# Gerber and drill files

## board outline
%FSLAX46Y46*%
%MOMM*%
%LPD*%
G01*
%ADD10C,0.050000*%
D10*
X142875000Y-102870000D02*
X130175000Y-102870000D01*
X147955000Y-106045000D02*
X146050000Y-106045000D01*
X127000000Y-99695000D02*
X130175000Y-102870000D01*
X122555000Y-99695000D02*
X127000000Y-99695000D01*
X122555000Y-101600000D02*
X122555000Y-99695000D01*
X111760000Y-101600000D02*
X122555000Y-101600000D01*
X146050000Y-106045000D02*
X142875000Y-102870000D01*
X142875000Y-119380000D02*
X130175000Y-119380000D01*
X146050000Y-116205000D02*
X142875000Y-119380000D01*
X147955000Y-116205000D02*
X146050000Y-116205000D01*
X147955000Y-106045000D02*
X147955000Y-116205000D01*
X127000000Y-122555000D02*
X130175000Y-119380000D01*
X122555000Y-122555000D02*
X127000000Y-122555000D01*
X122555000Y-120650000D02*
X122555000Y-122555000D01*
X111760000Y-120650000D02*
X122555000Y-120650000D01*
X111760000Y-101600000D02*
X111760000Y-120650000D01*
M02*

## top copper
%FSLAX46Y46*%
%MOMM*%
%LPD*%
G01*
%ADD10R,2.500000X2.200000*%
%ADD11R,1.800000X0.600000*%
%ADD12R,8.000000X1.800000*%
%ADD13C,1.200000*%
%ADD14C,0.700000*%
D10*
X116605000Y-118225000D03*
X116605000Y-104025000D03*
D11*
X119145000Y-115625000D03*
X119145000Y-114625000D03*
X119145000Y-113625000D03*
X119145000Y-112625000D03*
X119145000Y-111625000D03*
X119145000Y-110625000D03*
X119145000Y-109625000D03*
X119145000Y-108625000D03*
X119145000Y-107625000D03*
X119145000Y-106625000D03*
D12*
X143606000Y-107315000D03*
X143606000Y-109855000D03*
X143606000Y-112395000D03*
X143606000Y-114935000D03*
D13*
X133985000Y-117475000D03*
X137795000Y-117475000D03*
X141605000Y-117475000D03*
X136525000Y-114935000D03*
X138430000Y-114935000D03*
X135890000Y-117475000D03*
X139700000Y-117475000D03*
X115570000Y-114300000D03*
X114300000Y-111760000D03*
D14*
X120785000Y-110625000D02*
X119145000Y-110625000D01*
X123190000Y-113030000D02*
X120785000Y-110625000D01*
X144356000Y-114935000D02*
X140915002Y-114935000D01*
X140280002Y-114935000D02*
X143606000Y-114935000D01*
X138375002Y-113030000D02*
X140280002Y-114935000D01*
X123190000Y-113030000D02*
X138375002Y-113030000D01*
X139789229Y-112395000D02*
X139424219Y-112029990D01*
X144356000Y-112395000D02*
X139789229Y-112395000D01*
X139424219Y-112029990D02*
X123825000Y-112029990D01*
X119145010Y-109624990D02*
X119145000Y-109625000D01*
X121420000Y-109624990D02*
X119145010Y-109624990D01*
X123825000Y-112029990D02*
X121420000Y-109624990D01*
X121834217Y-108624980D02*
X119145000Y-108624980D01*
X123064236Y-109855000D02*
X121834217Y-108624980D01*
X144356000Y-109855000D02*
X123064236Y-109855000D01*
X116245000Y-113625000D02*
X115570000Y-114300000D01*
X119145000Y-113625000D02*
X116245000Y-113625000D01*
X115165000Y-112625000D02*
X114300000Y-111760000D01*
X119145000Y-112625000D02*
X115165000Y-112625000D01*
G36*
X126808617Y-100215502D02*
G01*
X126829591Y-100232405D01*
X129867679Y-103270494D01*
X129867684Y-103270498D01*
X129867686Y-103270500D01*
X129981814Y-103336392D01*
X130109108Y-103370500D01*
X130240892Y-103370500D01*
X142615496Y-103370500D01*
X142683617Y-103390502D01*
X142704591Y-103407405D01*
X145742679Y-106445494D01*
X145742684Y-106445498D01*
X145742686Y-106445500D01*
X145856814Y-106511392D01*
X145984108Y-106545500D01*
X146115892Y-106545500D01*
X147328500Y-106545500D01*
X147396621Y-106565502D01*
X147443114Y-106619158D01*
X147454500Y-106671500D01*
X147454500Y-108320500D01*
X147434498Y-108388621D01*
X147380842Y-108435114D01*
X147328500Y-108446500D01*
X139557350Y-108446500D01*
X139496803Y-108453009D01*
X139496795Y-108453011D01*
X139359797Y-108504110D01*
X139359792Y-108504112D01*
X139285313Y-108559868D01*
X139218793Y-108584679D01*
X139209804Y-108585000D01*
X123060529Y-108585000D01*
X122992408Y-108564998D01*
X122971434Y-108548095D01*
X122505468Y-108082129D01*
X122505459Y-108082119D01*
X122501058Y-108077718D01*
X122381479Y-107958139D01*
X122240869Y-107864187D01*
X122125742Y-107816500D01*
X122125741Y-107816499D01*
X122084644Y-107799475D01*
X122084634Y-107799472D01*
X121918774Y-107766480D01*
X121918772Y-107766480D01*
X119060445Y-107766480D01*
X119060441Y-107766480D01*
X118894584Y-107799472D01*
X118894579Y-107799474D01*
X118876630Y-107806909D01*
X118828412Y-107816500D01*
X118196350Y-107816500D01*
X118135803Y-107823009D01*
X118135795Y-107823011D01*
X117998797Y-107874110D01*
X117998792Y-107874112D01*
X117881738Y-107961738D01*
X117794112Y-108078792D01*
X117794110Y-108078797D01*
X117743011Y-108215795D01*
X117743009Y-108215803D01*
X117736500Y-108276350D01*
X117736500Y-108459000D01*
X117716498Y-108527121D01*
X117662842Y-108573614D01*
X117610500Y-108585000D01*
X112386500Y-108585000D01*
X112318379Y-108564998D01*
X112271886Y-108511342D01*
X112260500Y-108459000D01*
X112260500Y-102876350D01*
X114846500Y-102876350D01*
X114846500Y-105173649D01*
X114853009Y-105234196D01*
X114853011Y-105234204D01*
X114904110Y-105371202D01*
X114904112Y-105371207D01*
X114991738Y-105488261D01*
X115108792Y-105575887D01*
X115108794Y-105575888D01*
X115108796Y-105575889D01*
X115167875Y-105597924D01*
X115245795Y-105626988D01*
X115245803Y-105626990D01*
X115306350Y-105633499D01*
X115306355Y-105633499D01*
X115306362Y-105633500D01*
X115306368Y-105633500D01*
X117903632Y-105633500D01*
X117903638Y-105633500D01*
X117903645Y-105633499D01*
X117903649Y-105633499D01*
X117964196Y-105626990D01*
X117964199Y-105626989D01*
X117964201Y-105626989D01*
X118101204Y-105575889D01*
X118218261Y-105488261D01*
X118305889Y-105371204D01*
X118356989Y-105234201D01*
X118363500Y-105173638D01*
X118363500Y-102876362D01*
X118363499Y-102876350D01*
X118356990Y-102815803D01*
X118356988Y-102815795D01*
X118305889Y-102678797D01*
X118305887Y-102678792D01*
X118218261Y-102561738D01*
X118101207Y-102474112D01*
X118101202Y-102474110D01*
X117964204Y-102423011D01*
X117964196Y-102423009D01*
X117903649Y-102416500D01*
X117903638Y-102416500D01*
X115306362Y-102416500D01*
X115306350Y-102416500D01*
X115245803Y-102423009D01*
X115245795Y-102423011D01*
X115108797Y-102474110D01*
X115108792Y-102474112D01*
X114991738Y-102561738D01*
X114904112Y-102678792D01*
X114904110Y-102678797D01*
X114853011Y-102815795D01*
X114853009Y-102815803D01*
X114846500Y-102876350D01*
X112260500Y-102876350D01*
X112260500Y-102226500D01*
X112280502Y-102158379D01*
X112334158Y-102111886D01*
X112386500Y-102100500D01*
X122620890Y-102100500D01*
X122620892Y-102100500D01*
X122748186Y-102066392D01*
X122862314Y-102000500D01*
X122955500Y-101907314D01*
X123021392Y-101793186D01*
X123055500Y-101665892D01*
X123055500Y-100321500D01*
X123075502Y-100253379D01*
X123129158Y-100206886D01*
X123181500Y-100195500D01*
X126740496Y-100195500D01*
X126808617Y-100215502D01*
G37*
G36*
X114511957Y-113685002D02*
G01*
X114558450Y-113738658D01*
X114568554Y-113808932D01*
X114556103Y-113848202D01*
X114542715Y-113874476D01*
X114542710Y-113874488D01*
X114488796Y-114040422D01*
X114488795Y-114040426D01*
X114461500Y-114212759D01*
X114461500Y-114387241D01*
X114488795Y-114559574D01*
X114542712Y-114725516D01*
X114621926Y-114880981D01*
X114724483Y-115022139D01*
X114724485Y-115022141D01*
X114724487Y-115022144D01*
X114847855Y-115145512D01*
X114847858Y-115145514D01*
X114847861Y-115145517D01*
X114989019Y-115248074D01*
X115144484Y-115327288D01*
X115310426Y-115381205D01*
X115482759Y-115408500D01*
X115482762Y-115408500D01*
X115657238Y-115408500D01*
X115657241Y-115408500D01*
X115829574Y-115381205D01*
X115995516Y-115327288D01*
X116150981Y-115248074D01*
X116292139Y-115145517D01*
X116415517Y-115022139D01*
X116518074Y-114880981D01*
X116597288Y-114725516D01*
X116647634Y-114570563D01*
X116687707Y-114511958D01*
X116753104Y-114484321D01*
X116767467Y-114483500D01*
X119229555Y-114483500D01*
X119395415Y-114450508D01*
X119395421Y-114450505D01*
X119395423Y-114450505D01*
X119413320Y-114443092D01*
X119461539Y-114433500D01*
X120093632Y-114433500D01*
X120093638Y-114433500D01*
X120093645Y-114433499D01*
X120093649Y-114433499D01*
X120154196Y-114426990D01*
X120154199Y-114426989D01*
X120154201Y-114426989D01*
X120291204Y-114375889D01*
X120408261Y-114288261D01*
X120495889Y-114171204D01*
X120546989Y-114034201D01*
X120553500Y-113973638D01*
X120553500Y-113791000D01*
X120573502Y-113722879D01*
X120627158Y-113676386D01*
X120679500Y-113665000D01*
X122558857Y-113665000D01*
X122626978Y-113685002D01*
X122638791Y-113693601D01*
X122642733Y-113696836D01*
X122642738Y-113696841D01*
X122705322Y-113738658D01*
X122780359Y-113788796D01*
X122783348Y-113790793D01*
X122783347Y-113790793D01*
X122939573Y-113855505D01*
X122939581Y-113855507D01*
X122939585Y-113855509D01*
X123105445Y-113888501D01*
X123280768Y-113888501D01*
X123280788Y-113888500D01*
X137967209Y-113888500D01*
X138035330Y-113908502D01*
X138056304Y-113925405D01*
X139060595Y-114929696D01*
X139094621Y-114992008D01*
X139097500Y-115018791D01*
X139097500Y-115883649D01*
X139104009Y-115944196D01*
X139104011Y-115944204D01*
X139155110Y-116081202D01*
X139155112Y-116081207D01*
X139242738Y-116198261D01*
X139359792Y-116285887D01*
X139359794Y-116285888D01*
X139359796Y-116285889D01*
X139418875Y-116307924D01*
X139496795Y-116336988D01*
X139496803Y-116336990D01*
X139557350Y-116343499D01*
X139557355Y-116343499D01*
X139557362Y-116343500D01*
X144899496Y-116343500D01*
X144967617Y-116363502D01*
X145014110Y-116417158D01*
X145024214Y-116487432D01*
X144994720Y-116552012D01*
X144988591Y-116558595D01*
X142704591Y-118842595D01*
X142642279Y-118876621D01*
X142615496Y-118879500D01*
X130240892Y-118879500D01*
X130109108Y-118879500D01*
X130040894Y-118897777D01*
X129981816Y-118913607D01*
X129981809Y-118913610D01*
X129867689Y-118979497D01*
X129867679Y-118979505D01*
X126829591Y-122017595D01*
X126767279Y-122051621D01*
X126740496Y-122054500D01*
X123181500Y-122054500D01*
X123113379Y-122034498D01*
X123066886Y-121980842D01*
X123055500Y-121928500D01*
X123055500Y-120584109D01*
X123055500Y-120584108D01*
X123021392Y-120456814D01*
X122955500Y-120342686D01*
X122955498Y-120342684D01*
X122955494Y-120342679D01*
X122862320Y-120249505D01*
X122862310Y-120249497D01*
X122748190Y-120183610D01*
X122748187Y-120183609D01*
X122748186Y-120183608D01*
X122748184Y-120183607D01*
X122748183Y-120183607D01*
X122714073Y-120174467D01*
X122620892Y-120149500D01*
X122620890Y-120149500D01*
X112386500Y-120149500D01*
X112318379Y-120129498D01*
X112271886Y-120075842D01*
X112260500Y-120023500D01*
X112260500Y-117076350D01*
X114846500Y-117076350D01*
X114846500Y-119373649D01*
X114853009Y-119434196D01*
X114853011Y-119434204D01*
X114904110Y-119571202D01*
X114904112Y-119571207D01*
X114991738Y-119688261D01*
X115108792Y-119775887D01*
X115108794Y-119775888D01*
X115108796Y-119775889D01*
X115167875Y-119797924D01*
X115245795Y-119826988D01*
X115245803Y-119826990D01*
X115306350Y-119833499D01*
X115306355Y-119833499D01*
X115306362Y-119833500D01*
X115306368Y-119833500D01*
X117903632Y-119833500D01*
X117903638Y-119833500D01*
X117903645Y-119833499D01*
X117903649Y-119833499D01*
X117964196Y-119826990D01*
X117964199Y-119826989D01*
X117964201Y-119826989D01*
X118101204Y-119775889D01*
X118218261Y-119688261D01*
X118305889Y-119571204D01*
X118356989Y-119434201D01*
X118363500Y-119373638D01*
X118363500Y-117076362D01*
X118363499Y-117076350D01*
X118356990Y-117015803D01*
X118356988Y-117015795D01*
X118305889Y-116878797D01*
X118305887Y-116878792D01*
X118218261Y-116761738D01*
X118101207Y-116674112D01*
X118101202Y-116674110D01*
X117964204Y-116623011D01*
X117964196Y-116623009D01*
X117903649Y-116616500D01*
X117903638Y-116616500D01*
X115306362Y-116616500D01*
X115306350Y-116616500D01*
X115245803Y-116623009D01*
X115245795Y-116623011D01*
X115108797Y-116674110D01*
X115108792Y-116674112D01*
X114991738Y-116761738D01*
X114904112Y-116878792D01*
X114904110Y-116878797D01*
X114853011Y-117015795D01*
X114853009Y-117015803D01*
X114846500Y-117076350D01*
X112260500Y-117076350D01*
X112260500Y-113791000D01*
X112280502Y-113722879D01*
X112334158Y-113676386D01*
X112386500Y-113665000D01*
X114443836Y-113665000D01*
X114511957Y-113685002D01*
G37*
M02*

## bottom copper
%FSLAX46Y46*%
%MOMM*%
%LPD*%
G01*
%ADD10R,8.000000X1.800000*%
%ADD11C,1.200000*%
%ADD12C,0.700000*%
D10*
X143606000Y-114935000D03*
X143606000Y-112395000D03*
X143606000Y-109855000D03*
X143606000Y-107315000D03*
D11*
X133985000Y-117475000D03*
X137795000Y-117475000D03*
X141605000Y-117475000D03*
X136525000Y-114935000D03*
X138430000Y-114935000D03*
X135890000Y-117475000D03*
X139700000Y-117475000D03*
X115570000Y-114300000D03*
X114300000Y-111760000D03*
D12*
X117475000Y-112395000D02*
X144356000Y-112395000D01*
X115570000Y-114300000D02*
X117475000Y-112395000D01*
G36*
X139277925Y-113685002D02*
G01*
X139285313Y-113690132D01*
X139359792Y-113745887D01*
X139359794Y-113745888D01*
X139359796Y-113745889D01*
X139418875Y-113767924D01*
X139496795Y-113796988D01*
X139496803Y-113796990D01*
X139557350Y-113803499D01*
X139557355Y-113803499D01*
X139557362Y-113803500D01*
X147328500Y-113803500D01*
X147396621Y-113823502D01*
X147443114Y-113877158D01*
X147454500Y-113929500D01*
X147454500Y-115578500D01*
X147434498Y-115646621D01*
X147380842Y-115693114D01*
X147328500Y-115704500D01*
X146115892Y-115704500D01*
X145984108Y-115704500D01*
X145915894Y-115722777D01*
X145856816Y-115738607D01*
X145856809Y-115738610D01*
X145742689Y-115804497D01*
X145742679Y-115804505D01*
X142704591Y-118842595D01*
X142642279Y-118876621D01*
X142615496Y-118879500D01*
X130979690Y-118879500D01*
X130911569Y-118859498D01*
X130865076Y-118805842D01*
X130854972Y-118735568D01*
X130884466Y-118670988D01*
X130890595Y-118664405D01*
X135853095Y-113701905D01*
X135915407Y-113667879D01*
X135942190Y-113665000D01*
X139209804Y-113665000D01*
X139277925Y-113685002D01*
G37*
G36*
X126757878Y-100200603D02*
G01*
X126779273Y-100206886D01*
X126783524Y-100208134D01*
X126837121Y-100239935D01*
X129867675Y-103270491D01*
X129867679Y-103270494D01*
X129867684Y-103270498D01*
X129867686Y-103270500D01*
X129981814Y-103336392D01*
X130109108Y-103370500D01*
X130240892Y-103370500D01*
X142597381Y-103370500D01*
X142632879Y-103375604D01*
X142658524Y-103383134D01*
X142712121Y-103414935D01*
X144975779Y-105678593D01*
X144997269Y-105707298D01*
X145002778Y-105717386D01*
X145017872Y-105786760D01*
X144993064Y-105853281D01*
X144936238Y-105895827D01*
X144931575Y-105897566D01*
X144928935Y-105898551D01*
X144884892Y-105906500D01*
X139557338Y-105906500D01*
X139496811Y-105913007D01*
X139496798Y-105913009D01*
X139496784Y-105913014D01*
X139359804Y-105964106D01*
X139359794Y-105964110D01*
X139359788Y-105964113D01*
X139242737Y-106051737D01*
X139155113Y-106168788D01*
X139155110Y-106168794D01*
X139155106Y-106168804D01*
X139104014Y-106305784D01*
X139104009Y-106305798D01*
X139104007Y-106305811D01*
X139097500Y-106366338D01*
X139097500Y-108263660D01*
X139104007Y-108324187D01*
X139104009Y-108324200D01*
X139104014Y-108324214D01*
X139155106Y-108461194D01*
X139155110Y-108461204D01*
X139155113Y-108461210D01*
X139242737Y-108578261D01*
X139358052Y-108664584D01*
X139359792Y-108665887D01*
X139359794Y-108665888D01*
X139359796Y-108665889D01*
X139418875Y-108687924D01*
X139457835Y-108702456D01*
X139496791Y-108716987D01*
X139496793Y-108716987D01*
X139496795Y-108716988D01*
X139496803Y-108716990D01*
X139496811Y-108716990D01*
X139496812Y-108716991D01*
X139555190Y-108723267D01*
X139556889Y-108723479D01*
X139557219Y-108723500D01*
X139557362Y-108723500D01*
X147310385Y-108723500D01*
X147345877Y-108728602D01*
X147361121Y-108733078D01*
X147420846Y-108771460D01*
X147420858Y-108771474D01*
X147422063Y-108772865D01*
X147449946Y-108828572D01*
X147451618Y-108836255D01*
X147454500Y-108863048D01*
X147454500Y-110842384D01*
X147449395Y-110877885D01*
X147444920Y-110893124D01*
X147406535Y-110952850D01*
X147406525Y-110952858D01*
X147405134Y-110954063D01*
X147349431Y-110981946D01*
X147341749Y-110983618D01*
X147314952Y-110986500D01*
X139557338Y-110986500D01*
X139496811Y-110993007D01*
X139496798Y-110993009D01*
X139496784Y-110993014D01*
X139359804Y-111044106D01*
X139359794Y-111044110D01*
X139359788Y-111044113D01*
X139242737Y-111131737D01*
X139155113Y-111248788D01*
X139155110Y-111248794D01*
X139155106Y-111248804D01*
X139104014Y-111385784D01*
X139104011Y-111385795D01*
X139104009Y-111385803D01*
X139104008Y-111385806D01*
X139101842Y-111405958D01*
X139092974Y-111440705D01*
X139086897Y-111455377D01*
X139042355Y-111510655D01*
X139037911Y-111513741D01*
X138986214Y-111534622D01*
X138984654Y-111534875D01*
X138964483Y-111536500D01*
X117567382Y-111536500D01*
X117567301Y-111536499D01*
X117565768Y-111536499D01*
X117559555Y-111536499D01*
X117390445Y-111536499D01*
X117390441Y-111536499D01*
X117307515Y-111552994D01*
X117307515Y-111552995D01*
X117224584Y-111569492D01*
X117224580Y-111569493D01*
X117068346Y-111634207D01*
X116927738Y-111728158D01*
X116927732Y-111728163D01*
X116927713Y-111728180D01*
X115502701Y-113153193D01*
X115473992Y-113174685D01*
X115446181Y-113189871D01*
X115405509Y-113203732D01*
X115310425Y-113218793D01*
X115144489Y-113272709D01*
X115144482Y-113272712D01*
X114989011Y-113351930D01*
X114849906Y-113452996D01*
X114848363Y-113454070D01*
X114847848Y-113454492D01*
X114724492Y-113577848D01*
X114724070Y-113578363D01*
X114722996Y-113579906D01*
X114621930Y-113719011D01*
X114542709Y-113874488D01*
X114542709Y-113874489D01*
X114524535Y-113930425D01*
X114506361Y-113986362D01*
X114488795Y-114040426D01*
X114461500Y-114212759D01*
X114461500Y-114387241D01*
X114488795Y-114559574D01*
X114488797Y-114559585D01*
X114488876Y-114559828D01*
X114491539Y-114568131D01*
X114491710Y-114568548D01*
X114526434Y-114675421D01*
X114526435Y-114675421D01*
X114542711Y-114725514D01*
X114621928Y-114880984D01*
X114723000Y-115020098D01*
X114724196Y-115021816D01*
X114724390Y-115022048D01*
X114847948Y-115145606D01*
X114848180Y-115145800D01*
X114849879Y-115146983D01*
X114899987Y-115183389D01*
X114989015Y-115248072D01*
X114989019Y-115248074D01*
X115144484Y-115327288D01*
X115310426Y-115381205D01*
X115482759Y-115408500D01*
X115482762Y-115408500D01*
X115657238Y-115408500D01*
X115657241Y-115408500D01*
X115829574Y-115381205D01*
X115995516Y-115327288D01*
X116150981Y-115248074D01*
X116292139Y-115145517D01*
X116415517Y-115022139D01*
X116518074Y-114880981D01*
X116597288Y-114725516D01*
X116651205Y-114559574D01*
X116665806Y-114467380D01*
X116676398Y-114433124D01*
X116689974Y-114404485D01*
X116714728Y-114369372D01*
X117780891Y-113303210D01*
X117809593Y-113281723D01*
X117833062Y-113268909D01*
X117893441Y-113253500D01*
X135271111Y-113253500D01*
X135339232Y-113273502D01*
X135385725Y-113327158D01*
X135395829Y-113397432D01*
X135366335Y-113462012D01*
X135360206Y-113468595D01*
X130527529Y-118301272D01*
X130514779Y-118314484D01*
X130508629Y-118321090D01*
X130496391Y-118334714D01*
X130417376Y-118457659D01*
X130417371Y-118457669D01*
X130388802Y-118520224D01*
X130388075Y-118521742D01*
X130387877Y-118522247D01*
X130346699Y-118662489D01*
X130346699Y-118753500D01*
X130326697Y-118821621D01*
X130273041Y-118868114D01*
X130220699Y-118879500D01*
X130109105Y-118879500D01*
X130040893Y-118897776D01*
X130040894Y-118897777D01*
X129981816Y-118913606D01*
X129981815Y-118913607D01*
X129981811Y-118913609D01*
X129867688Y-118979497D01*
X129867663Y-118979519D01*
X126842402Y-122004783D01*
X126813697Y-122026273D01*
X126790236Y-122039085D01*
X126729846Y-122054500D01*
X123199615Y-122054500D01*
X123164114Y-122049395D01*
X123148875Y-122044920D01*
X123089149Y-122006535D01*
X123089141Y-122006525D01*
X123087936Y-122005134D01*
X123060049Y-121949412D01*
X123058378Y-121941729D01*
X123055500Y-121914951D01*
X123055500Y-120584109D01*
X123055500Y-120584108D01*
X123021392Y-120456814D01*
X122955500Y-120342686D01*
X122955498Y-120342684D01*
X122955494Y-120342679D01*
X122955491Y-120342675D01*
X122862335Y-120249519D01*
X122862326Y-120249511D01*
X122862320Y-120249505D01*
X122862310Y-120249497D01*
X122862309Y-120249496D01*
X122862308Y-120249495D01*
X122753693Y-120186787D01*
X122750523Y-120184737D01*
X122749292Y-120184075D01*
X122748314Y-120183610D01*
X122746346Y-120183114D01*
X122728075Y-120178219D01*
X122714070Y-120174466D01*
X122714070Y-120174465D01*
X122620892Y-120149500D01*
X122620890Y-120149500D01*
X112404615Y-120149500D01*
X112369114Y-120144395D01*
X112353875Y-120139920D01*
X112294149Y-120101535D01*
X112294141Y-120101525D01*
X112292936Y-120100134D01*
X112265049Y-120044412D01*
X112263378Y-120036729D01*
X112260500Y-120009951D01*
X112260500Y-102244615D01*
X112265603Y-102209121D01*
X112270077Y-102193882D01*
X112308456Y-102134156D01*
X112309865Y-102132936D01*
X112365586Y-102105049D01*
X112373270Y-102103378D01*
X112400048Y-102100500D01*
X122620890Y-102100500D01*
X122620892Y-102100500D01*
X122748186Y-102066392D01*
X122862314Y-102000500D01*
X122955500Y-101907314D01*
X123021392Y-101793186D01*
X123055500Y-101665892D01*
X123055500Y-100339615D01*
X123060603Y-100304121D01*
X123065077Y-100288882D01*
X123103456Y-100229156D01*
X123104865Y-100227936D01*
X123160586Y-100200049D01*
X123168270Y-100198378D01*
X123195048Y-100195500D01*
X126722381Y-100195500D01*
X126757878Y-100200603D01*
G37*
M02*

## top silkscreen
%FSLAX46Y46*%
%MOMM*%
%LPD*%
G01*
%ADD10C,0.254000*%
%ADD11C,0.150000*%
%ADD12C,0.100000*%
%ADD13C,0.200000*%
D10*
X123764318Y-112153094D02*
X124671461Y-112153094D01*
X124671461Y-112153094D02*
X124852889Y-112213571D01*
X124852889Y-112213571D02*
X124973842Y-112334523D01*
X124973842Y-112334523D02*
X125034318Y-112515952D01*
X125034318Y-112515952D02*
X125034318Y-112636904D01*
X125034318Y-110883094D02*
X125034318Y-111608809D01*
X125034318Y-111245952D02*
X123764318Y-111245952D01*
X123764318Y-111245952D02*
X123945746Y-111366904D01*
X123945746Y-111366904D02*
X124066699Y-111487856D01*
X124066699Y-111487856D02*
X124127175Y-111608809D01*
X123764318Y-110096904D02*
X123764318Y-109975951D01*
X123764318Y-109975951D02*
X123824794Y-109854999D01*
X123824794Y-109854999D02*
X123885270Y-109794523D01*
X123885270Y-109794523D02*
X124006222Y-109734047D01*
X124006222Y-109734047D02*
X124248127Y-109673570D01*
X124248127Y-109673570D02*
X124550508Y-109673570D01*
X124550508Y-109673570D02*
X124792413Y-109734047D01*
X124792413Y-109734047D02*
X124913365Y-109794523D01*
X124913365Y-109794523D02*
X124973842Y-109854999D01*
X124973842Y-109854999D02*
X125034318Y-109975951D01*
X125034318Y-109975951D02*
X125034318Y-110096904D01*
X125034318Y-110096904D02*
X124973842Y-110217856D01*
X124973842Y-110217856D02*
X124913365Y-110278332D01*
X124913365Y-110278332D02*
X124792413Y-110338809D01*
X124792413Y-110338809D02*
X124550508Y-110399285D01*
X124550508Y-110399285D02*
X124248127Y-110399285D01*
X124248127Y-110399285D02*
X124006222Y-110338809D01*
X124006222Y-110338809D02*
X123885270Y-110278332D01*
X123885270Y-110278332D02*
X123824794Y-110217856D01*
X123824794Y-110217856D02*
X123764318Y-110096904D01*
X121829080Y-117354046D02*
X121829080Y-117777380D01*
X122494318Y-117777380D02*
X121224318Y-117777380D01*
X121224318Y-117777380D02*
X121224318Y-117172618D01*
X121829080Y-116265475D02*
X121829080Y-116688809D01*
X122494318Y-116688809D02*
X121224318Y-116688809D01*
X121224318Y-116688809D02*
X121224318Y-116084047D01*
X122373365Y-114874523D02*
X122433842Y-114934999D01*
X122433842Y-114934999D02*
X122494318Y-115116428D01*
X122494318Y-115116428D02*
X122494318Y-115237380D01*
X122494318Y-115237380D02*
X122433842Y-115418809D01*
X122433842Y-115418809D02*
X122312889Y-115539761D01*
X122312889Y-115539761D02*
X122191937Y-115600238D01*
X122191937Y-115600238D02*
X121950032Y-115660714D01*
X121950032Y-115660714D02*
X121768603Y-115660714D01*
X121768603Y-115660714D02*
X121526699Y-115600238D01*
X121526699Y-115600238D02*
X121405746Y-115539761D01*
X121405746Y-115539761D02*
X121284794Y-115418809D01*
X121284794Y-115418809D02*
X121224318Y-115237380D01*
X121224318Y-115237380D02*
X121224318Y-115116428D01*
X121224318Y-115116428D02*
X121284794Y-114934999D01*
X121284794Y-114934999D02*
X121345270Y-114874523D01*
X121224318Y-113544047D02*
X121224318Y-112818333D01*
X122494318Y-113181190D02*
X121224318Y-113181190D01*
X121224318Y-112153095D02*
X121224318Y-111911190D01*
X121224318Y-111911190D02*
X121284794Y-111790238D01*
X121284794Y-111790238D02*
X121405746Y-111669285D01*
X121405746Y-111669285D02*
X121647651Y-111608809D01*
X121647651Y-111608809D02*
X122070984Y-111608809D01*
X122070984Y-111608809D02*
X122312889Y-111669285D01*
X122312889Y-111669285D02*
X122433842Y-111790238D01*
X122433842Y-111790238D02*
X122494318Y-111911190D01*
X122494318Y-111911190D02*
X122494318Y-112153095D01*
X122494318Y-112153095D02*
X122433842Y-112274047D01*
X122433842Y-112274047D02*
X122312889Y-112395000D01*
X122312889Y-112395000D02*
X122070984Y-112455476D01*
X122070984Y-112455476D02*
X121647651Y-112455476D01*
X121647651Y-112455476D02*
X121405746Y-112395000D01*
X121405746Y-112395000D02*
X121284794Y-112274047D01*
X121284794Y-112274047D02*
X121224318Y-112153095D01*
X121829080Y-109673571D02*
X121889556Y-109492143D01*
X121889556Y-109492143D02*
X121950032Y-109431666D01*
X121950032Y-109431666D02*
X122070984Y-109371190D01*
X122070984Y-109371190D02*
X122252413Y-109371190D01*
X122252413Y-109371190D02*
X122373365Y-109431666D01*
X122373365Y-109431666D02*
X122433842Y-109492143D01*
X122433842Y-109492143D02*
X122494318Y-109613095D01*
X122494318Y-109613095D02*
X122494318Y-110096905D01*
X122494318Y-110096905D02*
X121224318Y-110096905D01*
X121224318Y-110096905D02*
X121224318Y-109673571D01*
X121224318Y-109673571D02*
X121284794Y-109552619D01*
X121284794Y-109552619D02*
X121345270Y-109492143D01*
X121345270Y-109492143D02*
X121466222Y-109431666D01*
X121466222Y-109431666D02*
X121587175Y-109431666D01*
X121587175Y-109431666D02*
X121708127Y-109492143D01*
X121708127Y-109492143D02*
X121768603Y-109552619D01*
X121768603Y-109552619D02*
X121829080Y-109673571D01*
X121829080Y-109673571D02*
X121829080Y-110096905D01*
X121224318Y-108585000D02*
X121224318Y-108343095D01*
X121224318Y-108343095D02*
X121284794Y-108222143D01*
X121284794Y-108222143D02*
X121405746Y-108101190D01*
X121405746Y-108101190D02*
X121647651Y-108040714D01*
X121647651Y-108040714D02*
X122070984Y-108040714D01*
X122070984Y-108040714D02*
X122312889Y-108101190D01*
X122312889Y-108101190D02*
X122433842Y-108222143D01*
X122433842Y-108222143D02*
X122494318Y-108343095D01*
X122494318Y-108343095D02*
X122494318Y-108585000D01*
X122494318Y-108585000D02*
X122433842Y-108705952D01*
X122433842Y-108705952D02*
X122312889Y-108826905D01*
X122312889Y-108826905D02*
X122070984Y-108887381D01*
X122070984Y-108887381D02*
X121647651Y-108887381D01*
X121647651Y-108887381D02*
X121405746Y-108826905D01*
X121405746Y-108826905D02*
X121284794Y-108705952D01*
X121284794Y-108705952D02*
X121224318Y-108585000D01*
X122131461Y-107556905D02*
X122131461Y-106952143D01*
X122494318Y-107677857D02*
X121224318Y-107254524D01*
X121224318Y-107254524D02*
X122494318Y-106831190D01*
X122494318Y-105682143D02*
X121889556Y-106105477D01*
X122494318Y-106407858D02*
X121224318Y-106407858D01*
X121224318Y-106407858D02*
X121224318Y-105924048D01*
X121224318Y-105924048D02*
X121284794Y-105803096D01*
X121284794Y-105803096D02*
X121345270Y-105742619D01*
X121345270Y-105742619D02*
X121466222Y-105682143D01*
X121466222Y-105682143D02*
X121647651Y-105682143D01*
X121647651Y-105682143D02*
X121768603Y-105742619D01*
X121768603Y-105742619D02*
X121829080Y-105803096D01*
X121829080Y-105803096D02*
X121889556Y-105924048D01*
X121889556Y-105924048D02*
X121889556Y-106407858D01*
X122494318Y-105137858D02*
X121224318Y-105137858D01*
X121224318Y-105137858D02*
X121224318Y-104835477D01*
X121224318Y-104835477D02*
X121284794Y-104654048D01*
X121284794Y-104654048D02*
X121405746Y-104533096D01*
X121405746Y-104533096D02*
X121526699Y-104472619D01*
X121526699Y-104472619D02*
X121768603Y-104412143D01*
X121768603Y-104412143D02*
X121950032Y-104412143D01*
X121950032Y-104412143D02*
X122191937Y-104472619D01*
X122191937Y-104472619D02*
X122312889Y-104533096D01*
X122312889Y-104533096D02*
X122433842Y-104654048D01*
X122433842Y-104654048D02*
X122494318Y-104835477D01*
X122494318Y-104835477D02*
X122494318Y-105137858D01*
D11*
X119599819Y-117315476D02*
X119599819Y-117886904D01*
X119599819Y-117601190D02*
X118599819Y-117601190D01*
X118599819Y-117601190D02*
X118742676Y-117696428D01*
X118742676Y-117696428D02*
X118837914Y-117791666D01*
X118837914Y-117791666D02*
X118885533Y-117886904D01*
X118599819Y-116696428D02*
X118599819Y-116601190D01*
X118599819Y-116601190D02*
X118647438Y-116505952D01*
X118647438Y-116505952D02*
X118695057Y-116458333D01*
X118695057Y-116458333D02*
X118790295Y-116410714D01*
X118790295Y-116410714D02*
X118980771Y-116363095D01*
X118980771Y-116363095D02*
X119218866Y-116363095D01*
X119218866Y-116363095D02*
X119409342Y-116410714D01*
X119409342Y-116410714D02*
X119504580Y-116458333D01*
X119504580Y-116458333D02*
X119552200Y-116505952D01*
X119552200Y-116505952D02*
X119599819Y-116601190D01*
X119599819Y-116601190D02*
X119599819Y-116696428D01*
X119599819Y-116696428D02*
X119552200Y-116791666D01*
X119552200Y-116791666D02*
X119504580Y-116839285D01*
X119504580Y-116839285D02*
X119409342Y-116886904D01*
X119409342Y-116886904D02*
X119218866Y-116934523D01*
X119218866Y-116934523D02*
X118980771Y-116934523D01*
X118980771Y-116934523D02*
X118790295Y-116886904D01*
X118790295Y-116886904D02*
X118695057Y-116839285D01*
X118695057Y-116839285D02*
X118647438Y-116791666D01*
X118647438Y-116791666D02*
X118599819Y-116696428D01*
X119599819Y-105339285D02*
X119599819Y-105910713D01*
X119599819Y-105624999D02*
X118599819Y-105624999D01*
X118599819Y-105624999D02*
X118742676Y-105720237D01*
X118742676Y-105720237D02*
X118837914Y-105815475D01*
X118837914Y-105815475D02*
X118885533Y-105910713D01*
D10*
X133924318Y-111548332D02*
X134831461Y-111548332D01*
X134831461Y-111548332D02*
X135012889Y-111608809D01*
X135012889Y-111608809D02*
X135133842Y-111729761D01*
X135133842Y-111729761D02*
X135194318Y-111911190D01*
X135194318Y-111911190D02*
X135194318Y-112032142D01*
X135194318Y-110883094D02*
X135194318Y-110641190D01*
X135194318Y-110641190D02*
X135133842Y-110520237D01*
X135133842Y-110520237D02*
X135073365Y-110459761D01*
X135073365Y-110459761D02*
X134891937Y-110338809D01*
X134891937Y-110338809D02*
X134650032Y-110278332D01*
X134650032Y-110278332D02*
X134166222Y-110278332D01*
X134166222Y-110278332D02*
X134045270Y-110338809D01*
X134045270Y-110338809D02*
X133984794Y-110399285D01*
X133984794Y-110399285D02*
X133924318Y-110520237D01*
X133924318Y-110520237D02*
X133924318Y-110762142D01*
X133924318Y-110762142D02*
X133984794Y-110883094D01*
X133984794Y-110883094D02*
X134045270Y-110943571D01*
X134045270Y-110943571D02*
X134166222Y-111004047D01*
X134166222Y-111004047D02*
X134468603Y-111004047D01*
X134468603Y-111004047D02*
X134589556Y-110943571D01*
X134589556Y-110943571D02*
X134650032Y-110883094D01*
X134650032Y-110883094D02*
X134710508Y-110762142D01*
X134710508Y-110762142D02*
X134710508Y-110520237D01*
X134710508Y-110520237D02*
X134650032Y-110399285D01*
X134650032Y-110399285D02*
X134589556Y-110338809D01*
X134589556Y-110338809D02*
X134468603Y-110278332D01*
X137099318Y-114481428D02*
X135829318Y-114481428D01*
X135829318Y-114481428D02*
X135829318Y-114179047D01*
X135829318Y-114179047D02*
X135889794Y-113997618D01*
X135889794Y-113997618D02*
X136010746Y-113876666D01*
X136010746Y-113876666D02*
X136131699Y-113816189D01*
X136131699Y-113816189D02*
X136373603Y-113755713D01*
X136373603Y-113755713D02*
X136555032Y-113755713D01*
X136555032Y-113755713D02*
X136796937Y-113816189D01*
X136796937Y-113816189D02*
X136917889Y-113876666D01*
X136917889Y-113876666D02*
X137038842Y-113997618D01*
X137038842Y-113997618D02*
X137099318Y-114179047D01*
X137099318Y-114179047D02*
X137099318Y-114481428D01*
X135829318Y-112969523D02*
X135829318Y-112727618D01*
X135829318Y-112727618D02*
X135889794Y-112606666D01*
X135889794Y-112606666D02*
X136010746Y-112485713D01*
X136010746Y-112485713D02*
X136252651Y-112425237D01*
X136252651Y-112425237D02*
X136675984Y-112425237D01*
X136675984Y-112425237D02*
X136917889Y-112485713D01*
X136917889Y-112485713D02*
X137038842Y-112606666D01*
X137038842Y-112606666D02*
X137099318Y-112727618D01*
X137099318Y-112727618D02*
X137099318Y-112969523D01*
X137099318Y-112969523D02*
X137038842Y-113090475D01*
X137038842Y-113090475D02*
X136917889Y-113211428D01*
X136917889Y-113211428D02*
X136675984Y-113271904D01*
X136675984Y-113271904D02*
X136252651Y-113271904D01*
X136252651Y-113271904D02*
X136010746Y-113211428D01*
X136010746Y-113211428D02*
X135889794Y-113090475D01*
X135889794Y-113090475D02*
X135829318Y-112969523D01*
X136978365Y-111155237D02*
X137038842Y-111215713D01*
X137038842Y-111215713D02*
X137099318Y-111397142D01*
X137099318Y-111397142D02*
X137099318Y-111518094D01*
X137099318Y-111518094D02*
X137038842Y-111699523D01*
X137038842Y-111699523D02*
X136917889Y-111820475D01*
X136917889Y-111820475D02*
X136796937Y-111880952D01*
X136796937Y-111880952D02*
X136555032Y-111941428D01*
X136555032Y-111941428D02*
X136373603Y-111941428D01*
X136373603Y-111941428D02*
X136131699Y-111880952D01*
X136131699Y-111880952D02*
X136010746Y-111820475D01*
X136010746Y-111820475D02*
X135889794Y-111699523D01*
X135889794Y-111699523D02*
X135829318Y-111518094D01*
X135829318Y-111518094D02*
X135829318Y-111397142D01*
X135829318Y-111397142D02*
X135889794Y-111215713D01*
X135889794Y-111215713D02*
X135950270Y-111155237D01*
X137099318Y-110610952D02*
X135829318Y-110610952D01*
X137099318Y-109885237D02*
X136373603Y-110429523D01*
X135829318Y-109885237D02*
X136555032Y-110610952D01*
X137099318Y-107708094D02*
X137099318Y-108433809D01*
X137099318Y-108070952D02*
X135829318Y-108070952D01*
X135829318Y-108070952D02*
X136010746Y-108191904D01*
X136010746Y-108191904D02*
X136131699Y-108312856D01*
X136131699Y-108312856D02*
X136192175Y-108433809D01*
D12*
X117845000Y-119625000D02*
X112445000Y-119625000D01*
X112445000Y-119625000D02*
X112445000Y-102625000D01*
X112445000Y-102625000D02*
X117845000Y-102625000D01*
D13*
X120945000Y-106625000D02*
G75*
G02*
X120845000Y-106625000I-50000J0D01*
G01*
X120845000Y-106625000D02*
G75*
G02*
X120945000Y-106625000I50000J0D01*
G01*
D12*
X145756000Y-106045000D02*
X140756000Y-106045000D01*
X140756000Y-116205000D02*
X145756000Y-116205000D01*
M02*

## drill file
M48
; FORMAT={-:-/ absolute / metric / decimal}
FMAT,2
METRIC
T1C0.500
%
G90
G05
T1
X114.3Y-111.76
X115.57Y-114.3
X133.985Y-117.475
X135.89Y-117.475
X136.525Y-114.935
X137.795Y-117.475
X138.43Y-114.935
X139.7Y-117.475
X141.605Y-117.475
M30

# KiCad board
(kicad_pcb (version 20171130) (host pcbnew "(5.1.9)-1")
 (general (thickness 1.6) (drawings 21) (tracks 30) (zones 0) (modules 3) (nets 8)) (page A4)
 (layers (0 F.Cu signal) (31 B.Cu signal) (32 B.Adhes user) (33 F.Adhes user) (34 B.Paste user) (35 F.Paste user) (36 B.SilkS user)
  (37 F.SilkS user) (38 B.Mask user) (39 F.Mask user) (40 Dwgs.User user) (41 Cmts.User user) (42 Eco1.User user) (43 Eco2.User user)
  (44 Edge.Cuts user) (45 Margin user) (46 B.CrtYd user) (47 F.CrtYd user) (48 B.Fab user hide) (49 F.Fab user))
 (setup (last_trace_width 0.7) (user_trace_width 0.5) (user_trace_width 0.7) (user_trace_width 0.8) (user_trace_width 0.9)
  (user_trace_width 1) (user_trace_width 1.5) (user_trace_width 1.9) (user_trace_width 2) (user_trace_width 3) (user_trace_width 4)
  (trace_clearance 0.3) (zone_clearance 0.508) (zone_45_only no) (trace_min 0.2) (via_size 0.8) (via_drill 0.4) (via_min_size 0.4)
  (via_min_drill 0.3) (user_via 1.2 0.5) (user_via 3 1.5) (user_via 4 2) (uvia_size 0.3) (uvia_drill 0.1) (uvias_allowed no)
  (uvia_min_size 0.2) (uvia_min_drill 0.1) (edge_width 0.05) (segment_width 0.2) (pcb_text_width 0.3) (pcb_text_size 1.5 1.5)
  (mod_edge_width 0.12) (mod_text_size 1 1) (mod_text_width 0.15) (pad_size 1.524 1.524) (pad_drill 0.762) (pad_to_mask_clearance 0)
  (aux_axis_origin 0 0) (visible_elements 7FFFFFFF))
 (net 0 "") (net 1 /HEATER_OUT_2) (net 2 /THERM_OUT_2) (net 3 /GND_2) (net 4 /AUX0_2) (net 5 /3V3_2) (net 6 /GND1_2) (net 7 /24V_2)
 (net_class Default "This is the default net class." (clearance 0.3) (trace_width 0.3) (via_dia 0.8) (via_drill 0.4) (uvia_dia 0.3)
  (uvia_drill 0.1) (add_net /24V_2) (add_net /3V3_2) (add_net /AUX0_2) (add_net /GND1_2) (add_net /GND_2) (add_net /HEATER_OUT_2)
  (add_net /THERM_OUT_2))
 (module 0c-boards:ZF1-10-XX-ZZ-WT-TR (layer F.Cu) (at 119.145 111.125 270)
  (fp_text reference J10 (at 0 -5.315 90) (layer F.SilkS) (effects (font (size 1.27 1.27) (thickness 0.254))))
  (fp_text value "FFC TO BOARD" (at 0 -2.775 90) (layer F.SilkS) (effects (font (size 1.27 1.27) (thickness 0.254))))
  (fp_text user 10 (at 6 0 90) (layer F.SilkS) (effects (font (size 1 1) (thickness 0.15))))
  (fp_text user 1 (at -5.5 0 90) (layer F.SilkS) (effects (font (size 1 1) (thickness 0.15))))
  (fp_line (start 8.5 1.3) (end 8.5 6.7) (layer F.SilkS) (width 0.1))
  (fp_line (start 8.5 6.7) (end -8.5 6.7) (layer F.SilkS) (width 0.1))
  (fp_line (start -8.5 6.7) (end -8.5 1.3) (layer F.SilkS) (width 0.1))
  (fp_circle (center -4.5 -1.75) (end -4.5 -1.7) (layer F.SilkS) (width 0.2))
  (pad 12 smd rect (at 7.1 2.54 270) (size 2.2 2.5) (layers F.Cu F.Paste F.Mask))
  (pad 11 smd rect (at -7.1 2.54 270) (size 2.2 2.5) (layers F.Cu F.Paste F.Mask))
  (pad 10 smd rect (at 4.5 0 270) (size 0.6 1.8) (layers F.Cu F.Paste F.Mask) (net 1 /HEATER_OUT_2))
  (pad 9 smd rect (at 3.5 0 270) (size 0.6 1.8) (layers F.Cu F.Paste F.Mask) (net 1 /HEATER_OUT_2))
  (pad 8 smd rect (at 2.5 0 270) (size 0.6 1.8) (layers F.Cu F.Paste F.Mask) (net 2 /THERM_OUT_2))
  (pad 7 smd rect (at 1.5 0 270) (size 0.6 1.8) (layers F.Cu F.Paste F.Mask) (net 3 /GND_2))
  (pad 6 smd rect (at 0.5 0 270) (size 0.6 1.8) (layers F.Cu F.Paste F.Mask))
  (pad 5 smd rect (at -0.5 0 270) (size 0.6 1.8) (layers F.Cu F.Paste F.Mask) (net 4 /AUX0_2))
  (pad 4 smd rect (at -1.5 0 270) (size 0.6 1.8) (layers F.Cu F.Paste F.Mask) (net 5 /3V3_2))
  (pad 3 smd rect (at -2.5 0 270) (size 0.6 1.8) (layers F.Cu F.Paste F.Mask) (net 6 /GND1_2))
  (pad 2 smd rect (at -3.5 0 270) (size 0.6 1.8) (layers F.Cu F.Paste F.Mask) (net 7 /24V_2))
  (pad 1 smd rect (at -4.5 0 270) (size 0.6 1.8) (layers F.Cu F.Paste F.Mask) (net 7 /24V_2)))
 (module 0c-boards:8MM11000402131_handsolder (layer B.Cu) (at 144.145 111.125 90)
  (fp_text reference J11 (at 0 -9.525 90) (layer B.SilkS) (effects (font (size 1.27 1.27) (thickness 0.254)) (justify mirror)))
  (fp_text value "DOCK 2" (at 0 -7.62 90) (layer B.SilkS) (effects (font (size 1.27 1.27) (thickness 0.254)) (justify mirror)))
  (pad 1 smd rect (at -3.81 -0.539 90) (size 1.8 8) (layers B.Cu B.Paste B.Mask) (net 1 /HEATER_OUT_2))
  (pad 2 smd rect (at -1.27 -0.539 90) (size 1.8 8) (layers B.Cu B.Paste B.Mask) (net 2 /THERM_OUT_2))
  (pad 3 smd rect (at 1.27 -0.539 90) (size 1.8 8) (layers B.Cu B.Paste B.Mask) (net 3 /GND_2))
  (pad 4 smd rect (at 3.81 -0.539 90) (size 1.8 8) (layers B.Cu B.Paste B.Mask)))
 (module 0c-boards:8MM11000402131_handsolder (layer F.Cu) (at 144.145 111.125 270)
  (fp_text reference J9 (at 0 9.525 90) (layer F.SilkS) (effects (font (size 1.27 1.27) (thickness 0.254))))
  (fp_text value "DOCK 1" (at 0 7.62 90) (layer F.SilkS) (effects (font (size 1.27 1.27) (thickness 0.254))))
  (fp_line (start -5.08 -1.611) (end -5.08 3.389) (layer F.SilkS) (width 0.1))
  (fp_line (start 5.08 3.389) (end 5.08 -1.611) (layer F.SilkS) (width 0.1))
  (pad 1 smd rect (at -3.81 0.539 270) (size 1.8 8) (layers F.Cu F.Paste F.Mask) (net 7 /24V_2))
  (pad 2 smd rect (at -1.27 0.539 270) (size 1.8 8) (layers F.Cu F.Paste F.Mask) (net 6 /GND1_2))
  (pad 3 smd rect (at 1.27 0.539 270) (size 1.8 8) (layers F.Cu F.Paste F.Mask) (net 5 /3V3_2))
  (pad 4 smd rect (at 3.81 0.539 270) (size 1.8 8) (layers F.Cu F.Paste F.Mask) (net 4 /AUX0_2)))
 (gr_line (start 142.875 102.87) (end 130.175 102.87) (layer Edge.Cuts) (width 0.05))
 (gr_line (start 147.955 106.045) (end 146.05 106.045) (layer Edge.Cuts) (width 0.05))
 (gr_line (start 127 99.695) (end 130.175 102.87) (layer Edge.Cuts) (width 0.05))
 (gr_line (start 122.555 99.695) (end 127 99.695) (layer Edge.Cuts) (width 0.05))
 (gr_line (start 122.555 101.6) (end 122.555 99.695) (layer Edge.Cuts) (width 0.05))
 (gr_line (start 111.76 101.6) (end 122.555 101.6) (layer Edge.Cuts) (width 0.05))
 (gr_line (start 146.05 106.045) (end 142.875 102.87) (layer Edge.Cuts) (width 0.05))
 (gr_line (start 142.875 119.38) (end 130.175 119.38) (layer Edge.Cuts) (width 0.05))
 (gr_line (start 146.05 116.205) (end 142.875 119.38) (layer Edge.Cuts) (width 0.05))
 (gr_line (start 147.955 116.205) (end 146.05 116.205) (layer Edge.Cuts) (width 0.05))
 (gr_line (start 147.955 106.045) (end 147.955 116.205) (layer Edge.Cuts) (width 0.05))
 (gr_line (start 127 122.555) (end 130.175 119.38) (layer Edge.Cuts) (width 0.05))
 (gr_line (start 122.555 122.555) (end 127 122.555) (layer Edge.Cuts) (width 0.05))
 (gr_line (start 122.555 120.65) (end 122.555 122.555) (layer Edge.Cuts) (width 0.05))
 (gr_line (start 111.76 120.65) (end 122.555 120.65) (layer Edge.Cuts) (width 0.05))
 (gr_line (start 111.76 101.6) (end 111.76 120.65) (layer Edge.Cuts) (width 0.05))
 (segment (start 120.785 110.625) (end 119.145 110.625) (width 0.7) (layer F.Cu) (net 4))
 (segment (start 123.19 113.03) (end 120.785 110.625) (width 0.7) (layer F.Cu) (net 4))
 (segment (start 144.356 114.935) (end 140.915002 114.935) (width 0.7) (layer F.Cu) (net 4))
 (segment (start 140.280002 114.935) (end 143.606 114.935) (width 0.7) (layer F.Cu) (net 4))
 (segment (start 138.375002 113.03) (end 140.280002 114.935) (width 0.7) (layer F.Cu) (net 4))
 (segment (start 123.19 113.03) (end 138.375002 113.03) (width 0.7) (layer F.Cu) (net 4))
 (segment (start 139.789229 112.395) (end 139.424219 112.02999) (width 0.7) (layer F.Cu) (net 5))
 (segment (start 144.356 112.395) (end 139.789229 112.395) (width 0.7) (layer F.Cu) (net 5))
 (segment (start 139.424219 112.02999) (end 123.825 112.02999) (width 0.7) (layer F.Cu) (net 5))
 (segment (start 119.14501 109.62499) (end 119.145 109.625) (width 0.7) (layer F.Cu) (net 5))
 (segment (start 121.42 109.62499) (end 119.14501 109.62499) (width 0.7) (layer F.Cu) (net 5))
 (segment (start 123.825 112.02999) (end 121.42 109.62499) (width 0.7) (layer F.Cu) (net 5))
 (segment (start 121.834217 108.62498) (end 119.145 108.62498) (width 0.7) (layer F.Cu) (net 6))
 (segment (start 123.064236 109.855) (end 121.834217 108.62498) (width 0.7) (layer F.Cu) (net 6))
 (segment (start 144.356 109.855) (end 123.064236 109.855) (width 0.7) (layer F.Cu) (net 6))
 (via (at 133.985 117.475) (size 1.2) (drill 0.5) (layers F.Cu B.Cu) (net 1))
 (via (at 137.795 117.475) (size 1.2) (drill 0.5) (layers F.Cu B.Cu) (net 1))
 (via (at 141.605 117.475) (size 1.2) (drill 0.5) (layers F.Cu B.Cu) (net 1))
 (via (at 136.525 114.935) (size 1.2) (drill 0.5) (layers F.Cu B.Cu) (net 1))
 (via (at 138.43 114.935) (size 1.2) (drill 0.5) (layers F.Cu B.Cu) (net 1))
 (via (at 135.89 117.475) (size 1.2) (drill 0.5) (layers F.Cu B.Cu) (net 1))
 (via (at 139.7 117.475) (size 1.2) (drill 0.5) (layers F.Cu B.Cu) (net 1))
 (via (at 115.57 114.3) (size 1.2) (drill 0.5) (layers F.Cu B.Cu) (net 2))
 (segment (start 116.245 113.625) (end 115.57 114.3) (width 0.7) (layer F.Cu) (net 2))
 (segment (start 119.145 113.625) (end 116.245 113.625) (width 0.7) (layer F.Cu) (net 2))
 (segment (start 117.475 112.395) (end 144.356 112.395) (width 0.7) (layer B.Cu) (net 2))
 (segment (start 115.57 114.3) (end 117.475 112.395) (width 0.7) (layer B.Cu) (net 2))
 (via (at 114.3 111.76) (size 1.2) (drill 0.5) (layers F.Cu B.Cu) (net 3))
 (segment (start 115.165 112.625) (end 114.3 111.76) (width 0.7) (layer F.Cu) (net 3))
 (segment (start 119.145 112.625) (end 115.165 112.625) (width 0.7) (layer F.Cu) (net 3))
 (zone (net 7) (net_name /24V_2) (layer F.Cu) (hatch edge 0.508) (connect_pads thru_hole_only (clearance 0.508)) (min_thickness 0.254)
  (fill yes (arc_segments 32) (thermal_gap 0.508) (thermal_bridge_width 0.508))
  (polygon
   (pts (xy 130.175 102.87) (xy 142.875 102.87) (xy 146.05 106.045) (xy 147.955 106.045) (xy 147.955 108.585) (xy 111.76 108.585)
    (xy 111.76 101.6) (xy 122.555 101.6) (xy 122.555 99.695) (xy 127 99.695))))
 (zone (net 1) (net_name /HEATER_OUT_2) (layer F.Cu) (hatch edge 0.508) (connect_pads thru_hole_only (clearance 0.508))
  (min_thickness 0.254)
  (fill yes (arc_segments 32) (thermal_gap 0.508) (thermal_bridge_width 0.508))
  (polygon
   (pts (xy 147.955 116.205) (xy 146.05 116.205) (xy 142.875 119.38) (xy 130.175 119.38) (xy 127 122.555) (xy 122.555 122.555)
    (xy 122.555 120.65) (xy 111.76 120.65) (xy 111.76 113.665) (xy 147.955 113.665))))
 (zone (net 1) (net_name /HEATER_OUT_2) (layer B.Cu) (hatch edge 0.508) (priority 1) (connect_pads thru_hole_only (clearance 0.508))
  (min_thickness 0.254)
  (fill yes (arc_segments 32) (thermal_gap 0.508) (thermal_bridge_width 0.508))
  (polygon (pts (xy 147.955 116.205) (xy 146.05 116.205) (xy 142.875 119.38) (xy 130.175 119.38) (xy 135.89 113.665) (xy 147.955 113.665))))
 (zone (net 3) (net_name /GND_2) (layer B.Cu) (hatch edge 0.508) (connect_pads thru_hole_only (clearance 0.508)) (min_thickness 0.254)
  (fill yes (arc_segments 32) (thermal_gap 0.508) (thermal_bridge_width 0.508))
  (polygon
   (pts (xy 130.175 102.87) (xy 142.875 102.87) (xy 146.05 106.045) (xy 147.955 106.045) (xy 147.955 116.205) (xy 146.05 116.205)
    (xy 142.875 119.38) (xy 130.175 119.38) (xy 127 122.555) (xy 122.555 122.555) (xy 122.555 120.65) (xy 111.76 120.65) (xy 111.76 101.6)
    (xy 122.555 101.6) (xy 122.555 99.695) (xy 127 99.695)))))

